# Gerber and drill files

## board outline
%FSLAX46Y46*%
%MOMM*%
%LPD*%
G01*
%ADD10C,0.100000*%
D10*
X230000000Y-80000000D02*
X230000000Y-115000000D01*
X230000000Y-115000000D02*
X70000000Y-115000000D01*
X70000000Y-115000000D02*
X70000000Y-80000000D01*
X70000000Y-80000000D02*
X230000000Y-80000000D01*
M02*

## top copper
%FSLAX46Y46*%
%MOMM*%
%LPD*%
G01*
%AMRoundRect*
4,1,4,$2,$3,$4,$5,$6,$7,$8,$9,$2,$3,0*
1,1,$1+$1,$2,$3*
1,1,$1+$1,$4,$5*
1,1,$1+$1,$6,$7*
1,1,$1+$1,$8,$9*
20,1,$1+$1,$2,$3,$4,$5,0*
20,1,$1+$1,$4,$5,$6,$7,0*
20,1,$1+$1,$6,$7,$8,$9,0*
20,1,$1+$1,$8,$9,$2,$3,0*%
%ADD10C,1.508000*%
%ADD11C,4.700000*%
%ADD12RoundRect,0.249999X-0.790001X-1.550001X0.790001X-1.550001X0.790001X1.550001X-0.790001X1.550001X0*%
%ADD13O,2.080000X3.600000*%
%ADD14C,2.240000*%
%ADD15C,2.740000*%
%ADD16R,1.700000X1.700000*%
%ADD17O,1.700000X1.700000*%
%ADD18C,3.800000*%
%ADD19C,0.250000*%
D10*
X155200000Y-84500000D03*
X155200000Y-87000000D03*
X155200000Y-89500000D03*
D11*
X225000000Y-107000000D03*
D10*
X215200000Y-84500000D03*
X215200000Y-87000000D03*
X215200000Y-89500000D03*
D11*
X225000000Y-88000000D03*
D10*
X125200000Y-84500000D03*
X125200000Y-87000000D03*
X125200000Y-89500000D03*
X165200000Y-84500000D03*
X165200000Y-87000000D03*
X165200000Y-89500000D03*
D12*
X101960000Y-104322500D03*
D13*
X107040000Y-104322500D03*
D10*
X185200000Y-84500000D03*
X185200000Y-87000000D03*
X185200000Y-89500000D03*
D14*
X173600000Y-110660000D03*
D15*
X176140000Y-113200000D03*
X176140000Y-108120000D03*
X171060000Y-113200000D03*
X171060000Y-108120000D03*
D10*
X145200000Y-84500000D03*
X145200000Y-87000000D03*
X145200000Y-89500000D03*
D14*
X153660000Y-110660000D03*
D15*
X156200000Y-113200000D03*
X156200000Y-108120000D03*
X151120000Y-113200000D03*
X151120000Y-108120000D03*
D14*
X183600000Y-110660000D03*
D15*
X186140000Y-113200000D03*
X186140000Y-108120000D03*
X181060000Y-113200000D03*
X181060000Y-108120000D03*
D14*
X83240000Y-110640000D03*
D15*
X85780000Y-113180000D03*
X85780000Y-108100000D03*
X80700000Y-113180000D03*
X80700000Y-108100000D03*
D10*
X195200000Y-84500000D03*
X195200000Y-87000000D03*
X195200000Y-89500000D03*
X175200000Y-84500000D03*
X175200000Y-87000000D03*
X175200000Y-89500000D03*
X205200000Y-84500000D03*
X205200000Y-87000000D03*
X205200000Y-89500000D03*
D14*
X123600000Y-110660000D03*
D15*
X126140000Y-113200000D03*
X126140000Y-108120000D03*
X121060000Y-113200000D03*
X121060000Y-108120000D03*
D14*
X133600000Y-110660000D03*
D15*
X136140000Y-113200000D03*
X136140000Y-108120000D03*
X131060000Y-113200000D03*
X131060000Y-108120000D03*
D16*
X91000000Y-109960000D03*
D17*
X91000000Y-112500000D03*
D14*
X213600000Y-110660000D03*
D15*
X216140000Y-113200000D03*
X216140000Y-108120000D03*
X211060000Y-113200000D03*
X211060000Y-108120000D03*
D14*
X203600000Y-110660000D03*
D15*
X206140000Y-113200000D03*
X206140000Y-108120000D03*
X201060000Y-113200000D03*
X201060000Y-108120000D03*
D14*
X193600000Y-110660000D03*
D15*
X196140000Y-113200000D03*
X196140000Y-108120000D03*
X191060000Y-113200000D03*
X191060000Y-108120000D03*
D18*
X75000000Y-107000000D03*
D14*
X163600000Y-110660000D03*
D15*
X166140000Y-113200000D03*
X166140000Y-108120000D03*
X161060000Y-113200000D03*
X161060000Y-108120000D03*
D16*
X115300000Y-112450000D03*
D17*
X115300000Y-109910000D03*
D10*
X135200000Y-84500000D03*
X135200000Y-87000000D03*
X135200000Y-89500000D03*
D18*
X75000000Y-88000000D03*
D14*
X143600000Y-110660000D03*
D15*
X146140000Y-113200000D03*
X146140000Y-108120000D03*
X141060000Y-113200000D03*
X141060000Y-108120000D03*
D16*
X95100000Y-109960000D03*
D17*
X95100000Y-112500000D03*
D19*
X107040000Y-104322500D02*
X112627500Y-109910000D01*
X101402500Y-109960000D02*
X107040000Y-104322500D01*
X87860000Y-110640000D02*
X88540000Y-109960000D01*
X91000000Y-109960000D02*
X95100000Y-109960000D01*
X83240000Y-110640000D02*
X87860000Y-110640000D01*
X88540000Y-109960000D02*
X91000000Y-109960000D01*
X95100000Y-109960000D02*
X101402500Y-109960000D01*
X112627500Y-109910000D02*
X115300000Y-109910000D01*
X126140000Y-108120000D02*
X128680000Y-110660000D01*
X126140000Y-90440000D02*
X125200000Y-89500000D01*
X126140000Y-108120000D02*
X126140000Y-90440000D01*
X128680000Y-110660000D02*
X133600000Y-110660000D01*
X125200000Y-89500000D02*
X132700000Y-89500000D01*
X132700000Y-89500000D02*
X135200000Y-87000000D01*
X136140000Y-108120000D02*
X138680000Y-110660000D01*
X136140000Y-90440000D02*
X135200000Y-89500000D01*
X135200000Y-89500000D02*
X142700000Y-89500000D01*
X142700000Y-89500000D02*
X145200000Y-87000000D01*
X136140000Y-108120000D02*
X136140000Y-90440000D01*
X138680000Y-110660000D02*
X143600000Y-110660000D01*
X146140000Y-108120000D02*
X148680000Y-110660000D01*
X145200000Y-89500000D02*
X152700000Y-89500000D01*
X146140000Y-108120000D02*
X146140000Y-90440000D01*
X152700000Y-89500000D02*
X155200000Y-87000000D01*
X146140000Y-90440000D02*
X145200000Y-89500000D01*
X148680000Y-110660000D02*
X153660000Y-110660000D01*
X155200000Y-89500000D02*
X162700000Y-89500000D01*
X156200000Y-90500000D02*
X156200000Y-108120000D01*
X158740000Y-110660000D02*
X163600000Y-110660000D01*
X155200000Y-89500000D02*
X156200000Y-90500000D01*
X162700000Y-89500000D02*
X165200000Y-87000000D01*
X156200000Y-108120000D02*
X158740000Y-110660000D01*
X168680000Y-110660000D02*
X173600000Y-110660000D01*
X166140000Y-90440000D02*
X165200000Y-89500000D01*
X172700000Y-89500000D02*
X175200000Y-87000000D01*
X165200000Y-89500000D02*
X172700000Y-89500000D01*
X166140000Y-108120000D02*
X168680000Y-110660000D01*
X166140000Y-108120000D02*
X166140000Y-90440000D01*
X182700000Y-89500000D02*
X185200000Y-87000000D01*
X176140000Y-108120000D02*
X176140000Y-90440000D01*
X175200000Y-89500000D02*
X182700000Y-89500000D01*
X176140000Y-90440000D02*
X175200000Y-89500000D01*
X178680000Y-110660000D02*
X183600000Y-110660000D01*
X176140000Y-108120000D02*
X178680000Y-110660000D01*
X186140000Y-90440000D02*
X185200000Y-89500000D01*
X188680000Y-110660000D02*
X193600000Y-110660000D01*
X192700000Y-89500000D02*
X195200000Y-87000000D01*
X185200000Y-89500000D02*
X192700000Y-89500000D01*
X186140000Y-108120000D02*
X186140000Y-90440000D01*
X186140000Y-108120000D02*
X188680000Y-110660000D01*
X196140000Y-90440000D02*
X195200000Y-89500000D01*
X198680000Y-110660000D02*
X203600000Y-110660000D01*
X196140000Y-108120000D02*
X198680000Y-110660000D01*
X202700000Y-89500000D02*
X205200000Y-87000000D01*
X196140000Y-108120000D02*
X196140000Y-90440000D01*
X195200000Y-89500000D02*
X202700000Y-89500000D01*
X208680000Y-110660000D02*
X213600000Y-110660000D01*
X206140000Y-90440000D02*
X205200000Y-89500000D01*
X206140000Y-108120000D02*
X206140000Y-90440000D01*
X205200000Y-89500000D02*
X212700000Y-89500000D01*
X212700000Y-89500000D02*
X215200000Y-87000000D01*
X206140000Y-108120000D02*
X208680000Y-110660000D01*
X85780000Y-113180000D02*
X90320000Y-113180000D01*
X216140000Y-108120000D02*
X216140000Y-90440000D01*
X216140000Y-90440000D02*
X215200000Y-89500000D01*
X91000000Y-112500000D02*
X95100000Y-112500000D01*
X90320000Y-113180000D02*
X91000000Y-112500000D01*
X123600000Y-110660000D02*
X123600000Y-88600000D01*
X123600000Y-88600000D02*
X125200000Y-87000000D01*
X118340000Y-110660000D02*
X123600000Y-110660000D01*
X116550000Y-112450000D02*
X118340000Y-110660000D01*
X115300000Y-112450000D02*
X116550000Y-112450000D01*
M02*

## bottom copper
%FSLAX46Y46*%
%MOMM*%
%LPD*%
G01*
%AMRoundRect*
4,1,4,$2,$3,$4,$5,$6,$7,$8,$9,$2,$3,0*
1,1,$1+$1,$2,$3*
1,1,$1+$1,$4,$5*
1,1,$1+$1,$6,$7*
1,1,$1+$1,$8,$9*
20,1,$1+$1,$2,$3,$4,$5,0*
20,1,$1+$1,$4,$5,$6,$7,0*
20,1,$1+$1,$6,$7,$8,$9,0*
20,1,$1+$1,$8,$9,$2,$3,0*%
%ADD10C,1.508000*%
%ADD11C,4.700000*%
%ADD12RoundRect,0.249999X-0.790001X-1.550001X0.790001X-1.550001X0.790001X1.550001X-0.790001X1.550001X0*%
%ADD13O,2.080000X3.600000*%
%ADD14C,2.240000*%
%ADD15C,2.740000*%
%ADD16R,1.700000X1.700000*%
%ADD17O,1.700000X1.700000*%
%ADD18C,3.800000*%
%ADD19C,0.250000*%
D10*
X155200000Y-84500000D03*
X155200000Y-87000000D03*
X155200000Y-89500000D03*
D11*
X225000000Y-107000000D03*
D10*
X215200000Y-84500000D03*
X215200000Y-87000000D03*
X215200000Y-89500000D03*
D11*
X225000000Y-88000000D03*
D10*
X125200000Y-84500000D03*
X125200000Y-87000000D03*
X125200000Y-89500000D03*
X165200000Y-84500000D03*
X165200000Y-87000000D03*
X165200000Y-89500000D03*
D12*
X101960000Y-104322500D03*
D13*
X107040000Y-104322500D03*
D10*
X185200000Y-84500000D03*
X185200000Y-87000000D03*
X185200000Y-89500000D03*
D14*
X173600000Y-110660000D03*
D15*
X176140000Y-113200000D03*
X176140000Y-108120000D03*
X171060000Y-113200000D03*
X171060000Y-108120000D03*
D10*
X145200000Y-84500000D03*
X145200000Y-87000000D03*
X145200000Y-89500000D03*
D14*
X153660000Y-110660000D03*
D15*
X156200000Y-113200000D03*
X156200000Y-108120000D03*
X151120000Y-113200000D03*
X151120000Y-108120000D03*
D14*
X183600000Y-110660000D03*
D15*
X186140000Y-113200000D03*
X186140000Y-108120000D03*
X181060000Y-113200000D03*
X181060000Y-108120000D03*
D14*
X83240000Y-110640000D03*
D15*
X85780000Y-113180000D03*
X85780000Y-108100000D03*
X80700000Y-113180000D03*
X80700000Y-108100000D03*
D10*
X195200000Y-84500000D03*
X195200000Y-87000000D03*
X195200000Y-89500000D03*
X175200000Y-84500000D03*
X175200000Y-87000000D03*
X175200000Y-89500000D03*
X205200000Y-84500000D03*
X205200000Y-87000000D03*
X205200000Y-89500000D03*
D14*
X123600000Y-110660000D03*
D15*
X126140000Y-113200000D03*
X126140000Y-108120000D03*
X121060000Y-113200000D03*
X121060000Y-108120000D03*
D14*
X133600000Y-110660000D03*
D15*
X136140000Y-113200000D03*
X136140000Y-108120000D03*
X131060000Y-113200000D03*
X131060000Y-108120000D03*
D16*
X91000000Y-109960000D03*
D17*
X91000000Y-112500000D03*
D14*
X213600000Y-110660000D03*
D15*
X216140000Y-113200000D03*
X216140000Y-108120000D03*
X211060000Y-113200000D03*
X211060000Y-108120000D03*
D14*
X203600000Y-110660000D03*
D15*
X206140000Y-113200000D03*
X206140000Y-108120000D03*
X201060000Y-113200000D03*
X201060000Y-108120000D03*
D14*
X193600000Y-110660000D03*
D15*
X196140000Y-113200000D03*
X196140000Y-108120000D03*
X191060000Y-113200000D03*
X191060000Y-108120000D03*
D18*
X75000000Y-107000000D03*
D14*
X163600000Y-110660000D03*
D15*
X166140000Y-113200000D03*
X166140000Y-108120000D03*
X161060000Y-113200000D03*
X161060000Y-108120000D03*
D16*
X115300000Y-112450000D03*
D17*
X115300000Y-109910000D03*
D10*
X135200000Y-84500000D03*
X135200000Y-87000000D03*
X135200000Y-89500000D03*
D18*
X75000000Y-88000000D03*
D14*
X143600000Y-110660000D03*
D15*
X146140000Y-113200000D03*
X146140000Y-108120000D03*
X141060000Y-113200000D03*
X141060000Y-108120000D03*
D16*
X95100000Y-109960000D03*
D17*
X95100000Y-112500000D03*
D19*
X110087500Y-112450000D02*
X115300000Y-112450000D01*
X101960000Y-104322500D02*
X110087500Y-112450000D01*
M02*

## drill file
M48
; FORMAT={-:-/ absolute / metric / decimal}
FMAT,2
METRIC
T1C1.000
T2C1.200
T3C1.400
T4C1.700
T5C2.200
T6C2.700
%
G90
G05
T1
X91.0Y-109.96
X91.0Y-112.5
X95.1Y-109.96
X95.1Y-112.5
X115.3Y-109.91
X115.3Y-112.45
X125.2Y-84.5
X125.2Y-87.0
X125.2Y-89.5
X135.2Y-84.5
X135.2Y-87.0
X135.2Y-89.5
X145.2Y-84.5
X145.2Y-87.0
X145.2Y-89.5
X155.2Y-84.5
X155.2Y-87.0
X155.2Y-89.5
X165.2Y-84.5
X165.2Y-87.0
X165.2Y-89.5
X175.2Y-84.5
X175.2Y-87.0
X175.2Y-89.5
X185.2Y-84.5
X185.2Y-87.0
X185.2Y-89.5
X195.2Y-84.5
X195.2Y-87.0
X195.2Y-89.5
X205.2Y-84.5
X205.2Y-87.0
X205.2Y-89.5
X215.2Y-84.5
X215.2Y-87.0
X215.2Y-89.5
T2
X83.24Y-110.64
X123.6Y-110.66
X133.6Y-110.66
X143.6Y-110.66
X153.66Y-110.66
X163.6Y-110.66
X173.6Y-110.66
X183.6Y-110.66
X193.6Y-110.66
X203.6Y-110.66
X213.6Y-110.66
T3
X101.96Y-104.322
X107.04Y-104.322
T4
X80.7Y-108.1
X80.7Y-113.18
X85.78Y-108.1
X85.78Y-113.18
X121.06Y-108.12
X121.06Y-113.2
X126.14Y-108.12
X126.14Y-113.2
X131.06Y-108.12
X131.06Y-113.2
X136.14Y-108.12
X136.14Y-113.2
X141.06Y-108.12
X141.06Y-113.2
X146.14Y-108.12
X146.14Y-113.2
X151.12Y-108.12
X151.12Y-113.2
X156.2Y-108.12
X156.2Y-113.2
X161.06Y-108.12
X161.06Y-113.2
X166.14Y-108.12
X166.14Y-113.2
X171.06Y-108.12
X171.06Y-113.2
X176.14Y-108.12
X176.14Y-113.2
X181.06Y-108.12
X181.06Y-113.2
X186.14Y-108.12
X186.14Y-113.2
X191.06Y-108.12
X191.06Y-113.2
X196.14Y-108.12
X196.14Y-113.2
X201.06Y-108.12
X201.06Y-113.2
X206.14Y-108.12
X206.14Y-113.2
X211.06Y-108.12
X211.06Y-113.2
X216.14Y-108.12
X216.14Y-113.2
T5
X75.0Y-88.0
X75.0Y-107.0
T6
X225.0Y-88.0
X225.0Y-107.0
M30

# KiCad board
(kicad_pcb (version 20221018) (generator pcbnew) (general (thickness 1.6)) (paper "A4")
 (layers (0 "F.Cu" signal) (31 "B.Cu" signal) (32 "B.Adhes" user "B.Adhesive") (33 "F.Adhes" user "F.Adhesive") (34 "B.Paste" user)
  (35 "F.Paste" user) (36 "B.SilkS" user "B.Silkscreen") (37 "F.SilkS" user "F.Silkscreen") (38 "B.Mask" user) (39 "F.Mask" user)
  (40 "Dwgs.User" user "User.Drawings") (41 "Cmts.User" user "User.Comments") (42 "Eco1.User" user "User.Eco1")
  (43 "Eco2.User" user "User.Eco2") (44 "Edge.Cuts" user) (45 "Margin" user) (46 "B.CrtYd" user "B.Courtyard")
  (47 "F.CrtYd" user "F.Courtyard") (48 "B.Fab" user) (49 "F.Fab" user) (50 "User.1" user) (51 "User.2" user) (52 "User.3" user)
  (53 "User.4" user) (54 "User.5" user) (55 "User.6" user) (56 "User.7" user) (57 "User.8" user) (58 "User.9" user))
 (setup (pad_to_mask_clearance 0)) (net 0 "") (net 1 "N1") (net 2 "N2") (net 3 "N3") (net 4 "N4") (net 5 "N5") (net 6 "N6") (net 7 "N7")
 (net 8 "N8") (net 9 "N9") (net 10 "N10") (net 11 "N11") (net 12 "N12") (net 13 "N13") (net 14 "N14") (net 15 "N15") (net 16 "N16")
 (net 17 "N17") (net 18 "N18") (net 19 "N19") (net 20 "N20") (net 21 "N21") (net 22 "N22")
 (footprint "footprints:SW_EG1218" (layer "F.Cu") (at 155.2 87 -90)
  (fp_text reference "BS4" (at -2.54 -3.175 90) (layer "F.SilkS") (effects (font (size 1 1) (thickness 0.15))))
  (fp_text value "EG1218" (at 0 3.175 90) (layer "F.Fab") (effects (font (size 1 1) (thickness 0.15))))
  (pad "1" thru_hole circle (at -2.5 0 270) (size 1.508 1.508) (drill 1) (layers "*.Cu" "*.Mask") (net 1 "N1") (solder_mask_margin 0.102))
  (pad "2" thru_hole circle (at 0 0 270) (size 1.508 1.508) (drill 1) (layers "*.Cu" "*.Mask") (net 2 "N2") (solder_mask_margin 0.102))
  (pad "3" thru_hole circle (at 2.5 0 270) (size 1.508 1.508) (drill 1) (layers "*.Cu" "*.Mask") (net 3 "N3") (solder_mask_margin 0.102)))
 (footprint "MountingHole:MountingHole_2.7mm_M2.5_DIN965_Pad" (layer "F.Cu") (at 225 107)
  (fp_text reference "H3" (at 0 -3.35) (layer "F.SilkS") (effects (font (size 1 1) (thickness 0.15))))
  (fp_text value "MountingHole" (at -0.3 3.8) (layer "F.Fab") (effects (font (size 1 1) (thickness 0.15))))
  (pad "1" thru_hole circle (at 0 0) (size 4.7 4.7) (drill 2.7) (layers "*.Cu" "*.Mask")))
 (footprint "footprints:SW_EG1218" (layer "F.Cu") (at 215.2 87 -90)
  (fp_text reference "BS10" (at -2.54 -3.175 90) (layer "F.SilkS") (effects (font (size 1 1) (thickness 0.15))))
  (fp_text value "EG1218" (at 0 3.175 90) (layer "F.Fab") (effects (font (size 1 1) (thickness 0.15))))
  (pad "1" thru_hole circle (at -2.5 0 270) (size 1.508 1.508) (drill 1) (layers "*.Cu" "*.Mask") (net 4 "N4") (solder_mask_margin 0.102))
  (pad "2" thru_hole circle (at 0 0 270) (size 1.508 1.508) (drill 1) (layers "*.Cu" "*.Mask") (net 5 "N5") (solder_mask_margin 0.102))
  (pad "3" thru_hole circle (at 2.5 0 270) (size 1.508 1.508) (drill 1) (layers "*.Cu" "*.Mask") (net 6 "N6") (solder_mask_margin 0.102)))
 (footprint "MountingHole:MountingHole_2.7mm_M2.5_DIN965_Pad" (layer "F.Cu") (at 225 88)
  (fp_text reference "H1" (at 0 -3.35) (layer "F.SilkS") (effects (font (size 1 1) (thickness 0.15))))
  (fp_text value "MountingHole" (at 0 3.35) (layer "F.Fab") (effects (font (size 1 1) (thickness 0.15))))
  (pad "1" thru_hole circle (at 0 0) (size 4.7 4.7) (drill 2.7) (layers "*.Cu" "*.Mask")))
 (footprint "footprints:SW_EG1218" (layer "F.Cu") (at 125.2 87 -90)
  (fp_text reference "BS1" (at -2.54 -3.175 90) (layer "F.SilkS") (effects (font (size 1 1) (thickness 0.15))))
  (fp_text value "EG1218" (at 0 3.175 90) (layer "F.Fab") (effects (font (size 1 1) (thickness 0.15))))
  (pad "1" thru_hole circle (at -2.5 0 270) (size 1.508 1.508) (drill 1) (layers "*.Cu" "*.Mask") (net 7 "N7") (solder_mask_margin 0.102))
  (pad "2" thru_hole circle (at 0 0 270) (size 1.508 1.508) (drill 1) (layers "*.Cu" "*.Mask") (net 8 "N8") (solder_mask_margin 0.102))
  (pad "3" thru_hole circle (at 2.5 0 270) (size 1.508 1.508) (drill 1) (layers "*.Cu" "*.Mask") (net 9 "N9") (solder_mask_margin 0.102)))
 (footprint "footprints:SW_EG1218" (layer "F.Cu") (at 165.2 87 -90)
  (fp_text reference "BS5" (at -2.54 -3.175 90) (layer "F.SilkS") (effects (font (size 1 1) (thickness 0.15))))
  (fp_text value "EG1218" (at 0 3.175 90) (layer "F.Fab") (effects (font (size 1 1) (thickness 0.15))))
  (pad "1" thru_hole circle (at -2.5 0 270) (size 1.508 1.508) (drill 1) (layers "*.Cu" "*.Mask") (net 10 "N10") (solder_mask_margin 0.102))
  (pad "2" thru_hole circle (at 0 0 270) (size 1.508 1.508) (drill 1) (layers "*.Cu" "*.Mask") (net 3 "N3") (solder_mask_margin 0.102))
  (pad "3" thru_hole circle (at 2.5 0 270) (size 1.508 1.508) (drill 1) (layers "*.Cu" "*.Mask") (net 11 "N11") (solder_mask_margin 0.102)))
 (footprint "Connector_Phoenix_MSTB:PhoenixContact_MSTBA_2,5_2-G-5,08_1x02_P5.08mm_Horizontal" (layer "F.Cu") (at 101.96 104.3225)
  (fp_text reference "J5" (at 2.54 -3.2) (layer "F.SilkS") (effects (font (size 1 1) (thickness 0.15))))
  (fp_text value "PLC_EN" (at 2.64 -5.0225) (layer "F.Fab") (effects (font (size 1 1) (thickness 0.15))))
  (pad "1" thru_hole roundrect (at 0 0) (size 2.08 3.6) (drill 1.4) (layers "*.Cu" "*.Mask") (roundrect_rratio 0.1201918269) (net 8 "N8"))
  (pad "2" thru_hole oval (at 5.08 0) (size 2.08 3.6) (drill 1.4) (layers "*.Cu" "*.Mask") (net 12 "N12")))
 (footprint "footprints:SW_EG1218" (layer "F.Cu") (at 185.2 87 -90)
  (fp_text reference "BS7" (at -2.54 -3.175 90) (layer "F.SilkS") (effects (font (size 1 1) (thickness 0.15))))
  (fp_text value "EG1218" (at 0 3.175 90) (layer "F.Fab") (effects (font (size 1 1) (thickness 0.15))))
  (pad "1" thru_hole circle (at -2.5 0 270) (size 1.508 1.508) (drill 1) (layers "*.Cu" "*.Mask") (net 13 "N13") (solder_mask_margin 0.102))
  (pad "2" thru_hole circle (at 0 0 270) (size 1.508 1.508) (drill 1) (layers "*.Cu" "*.Mask") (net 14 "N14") (solder_mask_margin 0.102))
  (pad "3" thru_hole circle (at 2.5 0 270) (size 1.508 1.508) (drill 1) (layers "*.Cu" "*.Mask") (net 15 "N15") (solder_mask_margin 0.102)))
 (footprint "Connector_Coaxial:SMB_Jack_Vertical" (layer "F.Cu") (at 173.6 110.66 180)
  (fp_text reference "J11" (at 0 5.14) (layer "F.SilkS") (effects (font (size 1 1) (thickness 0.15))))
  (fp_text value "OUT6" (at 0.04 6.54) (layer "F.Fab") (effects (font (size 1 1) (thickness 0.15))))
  (pad "1" thru_hole circle (at 0 0 180) (size 2.24 2.24) (drill 1.2) (layers "*.Cu" "*.Mask") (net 11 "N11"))
  (pad "2" thru_hole circle (at -2.54 -2.54 180) (size 2.74 2.74) (drill 1.7) (layers "*.Cu" "*.Mask") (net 14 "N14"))
  (pad "2" thru_hole circle (at -2.54 2.54 180) (size 2.74 2.74) (drill 1.7) (layers "*.Cu" "*.Mask") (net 14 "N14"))
  (pad "2" thru_hole circle (at 2.54 -2.54 180) (size 2.74 2.74) (drill 1.7) (layers "*.Cu" "*.Mask") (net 14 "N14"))
  (pad "2" thru_hole circle (at 2.54 2.54 180) (size 2.74 2.74) (drill 1.7) (layers "*.Cu" "*.Mask") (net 14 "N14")))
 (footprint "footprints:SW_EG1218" (layer "F.Cu") (at 145.2 87 -90)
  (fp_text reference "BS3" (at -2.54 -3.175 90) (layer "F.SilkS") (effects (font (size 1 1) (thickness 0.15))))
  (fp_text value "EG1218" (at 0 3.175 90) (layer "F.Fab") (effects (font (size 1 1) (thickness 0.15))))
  (pad "1" thru_hole circle (at -2.5 0 270) (size 1.508 1.508) (drill 1) (layers "*.Cu" "*.Mask") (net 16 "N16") (solder_mask_margin 0.102))
  (pad "2" thru_hole circle (at 0 0 270) (size 1.508 1.508) (drill 1) (layers "*.Cu" "*.Mask") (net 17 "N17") (solder_mask_margin 0.102))
  (pad "3" thru_hole circle (at 2.5 0 270) (size 1.508 1.508) (drill 1) (layers "*.Cu" "*.Mask") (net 2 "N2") (solder_mask_margin 0.102)))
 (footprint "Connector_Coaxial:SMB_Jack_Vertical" (layer "F.Cu") (at 153.66 110.66 180)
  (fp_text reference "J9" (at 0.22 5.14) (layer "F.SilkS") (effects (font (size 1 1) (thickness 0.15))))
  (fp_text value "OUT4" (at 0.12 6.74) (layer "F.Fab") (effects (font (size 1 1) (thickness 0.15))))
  (pad "1" thru_hole circle (at 0 0 180) (size 2.24 2.24) (drill 1.2) (layers "*.Cu" "*.Mask") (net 2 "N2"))
  (pad "2" thru_hole circle (at -2.54 -2.54 180) (size 2.74 2.74) (drill 1.7) (layers "*.Cu" "*.Mask") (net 3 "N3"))
  (pad "2" thru_hole circle (at -2.54 2.54 180) (size 2.74 2.74) (drill 1.7) (layers "*.Cu" "*.Mask") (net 3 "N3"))
  (pad "2" thru_hole circle (at 2.54 -2.54 180) (size 2.74 2.74) (drill 1.7) (layers "*.Cu" "*.Mask") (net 3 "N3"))
  (pad "2" thru_hole circle (at 2.54 2.54 180) (size 2.74 2.74) (drill 1.7) (layers "*.Cu" "*.Mask") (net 3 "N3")))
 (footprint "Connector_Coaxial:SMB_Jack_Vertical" (layer "F.Cu") (at 183.6 110.66 180)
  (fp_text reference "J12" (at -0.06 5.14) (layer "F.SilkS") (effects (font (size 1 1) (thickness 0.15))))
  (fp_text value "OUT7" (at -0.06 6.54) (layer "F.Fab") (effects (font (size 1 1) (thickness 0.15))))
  (pad "1" thru_hole circle (at 0 0 180) (size 2.24 2.24) (drill 1.2) (layers "*.Cu" "*.Mask") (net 14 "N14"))
  (pad "2" thru_hole circle (at -2.54 -2.54 180) (size 2.74 2.74) (drill 1.7) (layers "*.Cu" "*.Mask") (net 15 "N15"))
  (pad "2" thru_hole circle (at -2.54 2.54 180) (size 2.74 2.74) (drill 1.7) (layers "*.Cu" "*.Mask") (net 15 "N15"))
  (pad "2" thru_hole circle (at 2.54 -2.54 180) (size 2.74 2.74) (drill 1.7) (layers "*.Cu" "*.Mask") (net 15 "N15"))
  (pad "2" thru_hole circle (at 2.54 2.54 180) (size 2.74 2.74) (drill 1.7) (layers "*.Cu" "*.Mask") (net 15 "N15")))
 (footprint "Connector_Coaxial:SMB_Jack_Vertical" (layer "F.Cu") (at 83.24 110.64 180)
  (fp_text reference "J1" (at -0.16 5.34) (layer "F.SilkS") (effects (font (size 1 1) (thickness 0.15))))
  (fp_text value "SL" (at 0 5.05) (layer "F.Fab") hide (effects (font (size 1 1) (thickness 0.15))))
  (pad "1" thru_hole circle (at 0 0 180) (size 2.24 2.24) (drill 1.2) (layers "*.Cu" "*.Mask") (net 12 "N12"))
  (pad "2" thru_hole circle (at -2.54 -2.54 180) (size 2.74 2.74) (drill 1.7) (layers "*.Cu" "*.Mask") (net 6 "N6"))
  (pad "2" thru_hole circle (at -2.54 2.54 180) (size 2.74 2.74) (drill 1.7) (layers "*.Cu" "*.Mask") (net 6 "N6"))
  (pad "2" thru_hole circle (at 2.54 -2.54 180) (size 2.74 2.74) (drill 1.7) (layers "*.Cu" "*.Mask") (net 6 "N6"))
  (pad "2" thru_hole circle (at 2.54 2.54 180) (size 2.74 2.74) (drill 1.7) (layers "*.Cu" "*.Mask") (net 6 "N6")))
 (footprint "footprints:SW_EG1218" (layer "F.Cu") (at 195.2 87 -90)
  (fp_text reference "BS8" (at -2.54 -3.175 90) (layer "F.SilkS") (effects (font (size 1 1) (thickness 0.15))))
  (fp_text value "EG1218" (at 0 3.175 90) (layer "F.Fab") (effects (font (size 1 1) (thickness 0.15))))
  (pad "1" thru_hole circle (at -2.5 0 270) (size 1.508 1.508) (drill 1) (layers "*.Cu" "*.Mask") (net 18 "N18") (solder_mask_margin 0.102))
  (pad "2" thru_hole circle (at 0 0 270) (size 1.508 1.508) (drill 1) (layers "*.Cu" "*.Mask") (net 15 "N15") (solder_mask_margin 0.102))
  (pad "3" thru_hole circle (at 2.5 0 270) (size 1.508 1.508) (drill 1) (layers "*.Cu" "*.Mask") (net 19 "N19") (solder_mask_margin 0.102)))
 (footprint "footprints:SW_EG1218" (layer "F.Cu") (at 175.2 87 -90)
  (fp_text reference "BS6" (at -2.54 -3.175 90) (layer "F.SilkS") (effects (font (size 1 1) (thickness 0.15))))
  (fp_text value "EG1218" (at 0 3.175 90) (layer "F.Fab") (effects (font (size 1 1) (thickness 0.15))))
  (pad "1" thru_hole circle (at -2.5 0 270) (size 1.508 1.508) (drill 1) (layers "*.Cu" "*.Mask") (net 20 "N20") (solder_mask_margin 0.102))
  (pad "2" thru_hole circle (at 0 0 270) (size 1.508 1.508) (drill 1) (layers "*.Cu" "*.Mask") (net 11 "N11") (solder_mask_margin 0.102))
  (pad "3" thru_hole circle (at 2.5 0 270) (size 1.508 1.508) (drill 1) (layers "*.Cu" "*.Mask") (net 14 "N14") (solder_mask_margin 0.102)))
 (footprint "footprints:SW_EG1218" (layer "F.Cu") (at 205.2 87 -90)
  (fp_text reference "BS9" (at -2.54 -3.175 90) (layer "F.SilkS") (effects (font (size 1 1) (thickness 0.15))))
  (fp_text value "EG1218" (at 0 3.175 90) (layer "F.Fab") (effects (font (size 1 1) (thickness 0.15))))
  (pad "1" thru_hole circle (at -2.5 0 270) (size 1.508 1.508) (drill 1) (layers "*.Cu" "*.Mask") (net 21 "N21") (solder_mask_margin 0.102))
  (pad "2" thru_hole circle (at 0 0 270) (size 1.508 1.508) (drill 1) (layers "*.Cu" "*.Mask") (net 19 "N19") (solder_mask_margin 0.102))
  (pad "3" thru_hole circle (at 2.5 0 270) (size 1.508 1.508) (drill 1) (layers "*.Cu" "*.Mask") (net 5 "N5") (solder_mask_margin 0.102)))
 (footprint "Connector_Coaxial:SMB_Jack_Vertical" (layer "F.Cu") (at 123.6 110.66 180)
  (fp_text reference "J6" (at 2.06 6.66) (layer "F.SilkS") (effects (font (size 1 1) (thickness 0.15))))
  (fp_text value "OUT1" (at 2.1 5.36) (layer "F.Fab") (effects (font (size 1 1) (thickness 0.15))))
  (pad "1" thru_hole circle (at 0 0 180) (size 2.24 2.24) (drill 1.2) (layers "*.Cu" "*.Mask") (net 8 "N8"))
  (pad "2" thru_hole circle (at -2.54 -2.54 180) (size 2.74 2.74) (drill 1.7) (layers "*.Cu" "*.Mask") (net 9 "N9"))
  (pad "2" thru_hole circle (at -2.54 2.54 180) (size 2.74 2.74) (drill 1.7) (layers "*.Cu" "*.Mask") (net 9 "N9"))
  (pad "2" thru_hole circle (at 2.54 -2.54 180) (size 2.74 2.74) (drill 1.7) (layers "*.Cu" "*.Mask") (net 9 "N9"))
  (pad "2" thru_hole circle (at 2.54 2.54 180) (size 2.74 2.74) (drill 1.7) (layers "*.Cu" "*.Mask") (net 9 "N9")))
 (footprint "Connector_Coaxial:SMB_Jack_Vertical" (layer "F.Cu") (at 133.6 110.66 180)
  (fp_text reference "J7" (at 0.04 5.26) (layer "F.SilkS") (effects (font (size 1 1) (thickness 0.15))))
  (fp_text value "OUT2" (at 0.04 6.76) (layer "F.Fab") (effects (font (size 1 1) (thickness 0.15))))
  (pad "1" thru_hole circle (at 0 0 180) (size 2.24 2.24) (drill 1.2) (layers "*.Cu" "*.Mask") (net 9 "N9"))
  (pad "2" thru_hole circle (at -2.54 -2.54 180) (size 2.74 2.74) (drill 1.7) (layers "*.Cu" "*.Mask") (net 17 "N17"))
  (pad "2" thru_hole circle (at -2.54 2.54 180) (size 2.74 2.74) (drill 1.7) (layers "*.Cu" "*.Mask") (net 17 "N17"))
  (pad "2" thru_hole circle (at 2.54 -2.54 180) (size 2.74 2.74) (drill 1.7) (layers "*.Cu" "*.Mask") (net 17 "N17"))
  (pad "2" thru_hole circle (at 2.54 2.54 180) (size 2.74 2.74) (drill 1.7) (layers "*.Cu" "*.Mask") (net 17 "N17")))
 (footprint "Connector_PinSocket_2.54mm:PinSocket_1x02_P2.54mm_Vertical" (layer "F.Cu") (at 91 109.96)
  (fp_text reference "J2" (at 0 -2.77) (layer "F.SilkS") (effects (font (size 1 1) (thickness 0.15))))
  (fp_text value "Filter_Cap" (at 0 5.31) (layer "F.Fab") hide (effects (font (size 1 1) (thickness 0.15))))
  (pad "1" thru_hole rect (at 0 0) (size 1.7 1.7) (drill 1) (layers "*.Cu" "*.Mask") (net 12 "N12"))
  (pad "2" thru_hole oval (at 0 2.54) (size 1.7 1.7) (drill 1) (layers "*.Cu" "*.Mask") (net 6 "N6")))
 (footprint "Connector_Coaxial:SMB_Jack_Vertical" (layer "F.Cu") (at 213.6 110.66 180)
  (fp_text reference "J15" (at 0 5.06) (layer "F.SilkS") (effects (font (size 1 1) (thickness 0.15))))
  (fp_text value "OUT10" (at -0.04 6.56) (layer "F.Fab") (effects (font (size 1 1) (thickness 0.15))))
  (pad "1" thru_hole circle (at 0 0 180) (size 2.24 2.24) (drill 1.2) (layers "*.Cu" "*.Mask") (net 5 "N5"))
  (pad "2" thru_hole circle (at -2.54 -2.54 180) (size 2.74 2.74) (drill 1.7) (layers "*.Cu" "*.Mask") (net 6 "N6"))
  (pad "2" thru_hole circle (at -2.54 2.54 180) (size 2.74 2.74) (drill 1.7) (layers "*.Cu" "*.Mask") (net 6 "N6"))
  (pad "2" thru_hole circle (at 2.54 -2.54 180) (size 2.74 2.74) (drill 1.7) (layers "*.Cu" "*.Mask") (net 6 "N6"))
  (pad "2" thru_hole circle (at 2.54 2.54 180) (size 2.74 2.74) (drill 1.7) (layers "*.Cu" "*.Mask") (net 6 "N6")))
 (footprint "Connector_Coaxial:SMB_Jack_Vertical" (layer "F.Cu") (at 203.6 110.66 180)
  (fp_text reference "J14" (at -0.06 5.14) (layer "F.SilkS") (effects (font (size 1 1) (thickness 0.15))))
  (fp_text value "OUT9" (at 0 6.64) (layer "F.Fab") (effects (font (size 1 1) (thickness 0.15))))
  (pad "1" thru_hole circle (at 0 0 180) (size 2.24 2.24) (drill 1.2) (layers "*.Cu" "*.Mask") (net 19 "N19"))
  (pad "2" thru_hole circle (at -2.54 -2.54 180) (size 2.74 2.74) (drill 1.7) (layers "*.Cu" "*.Mask") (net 5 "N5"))
  (pad "2" thru_hole circle (at -2.54 2.54 180) (size 2.74 2.74) (drill 1.7) (layers "*.Cu" "*.Mask") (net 5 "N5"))
  (pad "2" thru_hole circle (at 2.54 -2.54 180) (size 2.74 2.74) (drill 1.7) (layers "*.Cu" "*.Mask") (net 5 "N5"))
  (pad "2" thru_hole circle (at 2.54 2.54 180) (size 2.74 2.74) (drill 1.7) (layers "*.Cu" "*.Mask") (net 5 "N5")))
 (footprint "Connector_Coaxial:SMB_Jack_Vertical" (layer "F.Cu") (at 193.6 110.66 180)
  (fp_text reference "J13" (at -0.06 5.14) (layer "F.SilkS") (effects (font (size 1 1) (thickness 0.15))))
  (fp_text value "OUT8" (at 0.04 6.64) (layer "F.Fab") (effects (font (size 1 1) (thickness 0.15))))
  (pad "1" thru_hole circle (at 0 0 180) (size 2.24 2.24) (drill 1.2) (layers "*.Cu" "*.Mask") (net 15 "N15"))
  (pad "2" thru_hole circle (at -2.54 -2.54 180) (size 2.74 2.74) (drill 1.7) (layers "*.Cu" "*.Mask") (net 19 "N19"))
  (pad "2" thru_hole circle (at -2.54 2.54 180) (size 2.74 2.74) (drill 1.7) (layers "*.Cu" "*.Mask") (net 19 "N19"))
  (pad "2" thru_hole circle (at 2.54 -2.54 180) (size 2.74 2.74) (drill 1.7) (layers "*.Cu" "*.Mask") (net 19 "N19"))
  (pad "2" thru_hole circle (at 2.54 2.54 180) (size 2.74 2.74) (drill 1.7) (layers "*.Cu" "*.Mask") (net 19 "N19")))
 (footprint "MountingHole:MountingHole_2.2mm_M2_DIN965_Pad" (layer "F.Cu") (at 75 107)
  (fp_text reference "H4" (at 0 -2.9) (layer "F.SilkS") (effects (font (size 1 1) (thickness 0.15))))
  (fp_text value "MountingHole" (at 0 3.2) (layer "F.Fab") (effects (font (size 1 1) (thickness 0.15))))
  (pad "1" thru_hole circle (at 0 0) (size 3.8 3.8) (drill 2.2) (layers "*.Cu" "*.Mask")))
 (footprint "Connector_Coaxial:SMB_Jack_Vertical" (layer "F.Cu") (at 163.6 110.66 180)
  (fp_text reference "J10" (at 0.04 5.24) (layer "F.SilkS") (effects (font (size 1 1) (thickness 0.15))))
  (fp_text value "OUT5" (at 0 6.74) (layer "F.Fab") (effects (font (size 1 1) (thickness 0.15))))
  (pad "1" thru_hole circle (at 0 0 180) (size 2.24 2.24) (drill 1.2) (layers "*.Cu" "*.Mask") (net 3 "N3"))
  (pad "2" thru_hole circle (at -2.54 -2.54 180) (size 2.74 2.74) (drill 1.7) (layers "*.Cu" "*.Mask") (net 11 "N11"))
  (pad "2" thru_hole circle (at -2.54 2.54 180) (size 2.74 2.74) (drill 1.7) (layers "*.Cu" "*.Mask") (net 11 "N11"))
  (pad "2" thru_hole circle (at 2.54 -2.54 180) (size 2.74 2.74) (drill 1.7) (layers "*.Cu" "*.Mask") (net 11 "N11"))
  (pad "2" thru_hole circle (at 2.54 2.54 180) (size 2.74 2.74) (drill 1.7) (layers "*.Cu" "*.Mask") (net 11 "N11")))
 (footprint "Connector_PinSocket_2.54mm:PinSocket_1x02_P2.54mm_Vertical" (layer "F.Cu") (at 115.3 112.45 180)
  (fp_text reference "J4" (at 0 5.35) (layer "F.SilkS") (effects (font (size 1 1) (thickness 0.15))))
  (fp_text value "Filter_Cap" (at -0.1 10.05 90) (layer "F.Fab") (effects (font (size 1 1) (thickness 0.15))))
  (pad "1" thru_hole rect (at 0 0 180) (size 1.7 1.7) (drill 1) (layers "*.Cu" "*.Mask") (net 8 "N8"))
  (pad "2" thru_hole oval (at 0 2.54 180) (size 1.7 1.7) (drill 1) (layers "*.Cu" "*.Mask") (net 12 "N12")))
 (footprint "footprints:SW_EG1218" (layer "F.Cu") (at 135.2 87 -90)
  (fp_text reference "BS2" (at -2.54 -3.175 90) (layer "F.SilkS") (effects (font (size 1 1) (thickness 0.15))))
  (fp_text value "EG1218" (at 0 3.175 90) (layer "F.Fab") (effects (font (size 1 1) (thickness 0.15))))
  (pad "1" thru_hole circle (at -2.5 0 270) (size 1.508 1.508) (drill 1) (layers "*.Cu" "*.Mask") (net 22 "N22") (solder_mask_margin 0.102))
  (pad "2" thru_hole circle (at 0 0 270) (size 1.508 1.508) (drill 1) (layers "*.Cu" "*.Mask") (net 9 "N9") (solder_mask_margin 0.102))
  (pad "3" thru_hole circle (at 2.5 0 270) (size 1.508 1.508) (drill 1) (layers "*.Cu" "*.Mask") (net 17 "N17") (solder_mask_margin 0.102)))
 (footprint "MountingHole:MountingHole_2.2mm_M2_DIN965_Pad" (layer "F.Cu") (at 75 88)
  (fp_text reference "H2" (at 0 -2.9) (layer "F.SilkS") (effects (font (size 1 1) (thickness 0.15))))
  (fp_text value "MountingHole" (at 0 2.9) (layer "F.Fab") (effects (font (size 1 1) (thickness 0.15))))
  (pad "1" thru_hole circle (at 0 0) (size 3.8 3.8) (drill 2.2) (layers "*.Cu" "*.Mask")))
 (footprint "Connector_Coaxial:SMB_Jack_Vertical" (layer "F.Cu") (at 143.6 110.66 180)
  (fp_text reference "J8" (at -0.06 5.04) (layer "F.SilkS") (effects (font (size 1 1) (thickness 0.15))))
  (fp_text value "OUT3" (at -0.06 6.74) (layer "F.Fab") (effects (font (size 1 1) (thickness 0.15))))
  (pad "1" thru_hole circle (at 0 0 180) (size 2.24 2.24) (drill 1.2) (layers "*.Cu" "*.Mask") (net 17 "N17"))
  (pad "2" thru_hole circle (at -2.54 -2.54 180) (size 2.74 2.74) (drill 1.7) (layers "*.Cu" "*.Mask") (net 2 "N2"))
  (pad "2" thru_hole circle (at -2.54 2.54 180) (size 2.74 2.74) (drill 1.7) (layers "*.Cu" "*.Mask") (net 2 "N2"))
  (pad "2" thru_hole circle (at 2.54 -2.54 180) (size 2.74 2.74) (drill 1.7) (layers "*.Cu" "*.Mask") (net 2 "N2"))
  (pad "2" thru_hole circle (at 2.54 2.54 180) (size 2.74 2.74) (drill 1.7) (layers "*.Cu" "*.Mask") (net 2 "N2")))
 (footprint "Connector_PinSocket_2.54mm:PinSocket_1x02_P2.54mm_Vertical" (layer "F.Cu") (at 95.1 109.96)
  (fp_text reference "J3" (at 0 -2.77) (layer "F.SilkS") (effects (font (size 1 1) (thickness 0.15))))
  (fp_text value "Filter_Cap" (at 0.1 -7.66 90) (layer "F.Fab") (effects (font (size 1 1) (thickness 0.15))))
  (pad "1" thru_hole rect (at 0 0) (size 1.7 1.7) (drill 1) (layers "*.Cu" "*.Mask") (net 12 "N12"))
  (pad "2" thru_hole oval (at 0 2.54) (size 1.7 1.7) (drill 1) (layers "*.Cu" "*.Mask") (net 6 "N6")))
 (gr_line (start 230 80) (end 230 115) (stroke (width 0.1) (type default)) (layer "Edge.Cuts"))
 (gr_line (start 230 115) (end 70 115) (stroke (width 0.1) (type default)) (layer "Edge.Cuts"))
 (gr_line (start 70 115) (end 70 80) (stroke (width 0.1) (type default)) (layer "Edge.Cuts"))
 (gr_line (start 70 80) (end 230 80) (stroke (width 0.1) (type default)) (layer "Edge.Cuts"))
 (segment (start 107.04 104.3225) (end 112.6275 109.91) (width 0.25) (layer "F.Cu") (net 12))
 (segment (start 101.4025 109.96) (end 107.04 104.3225) (width 0.25) (layer "F.Cu") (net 12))
 (segment (start 87.86 110.64) (end 88.54 109.96) (width 0.25) (layer "F.Cu") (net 12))
 (segment (start 91 109.96) (end 95.1 109.96) (width 0.25) (layer "F.Cu") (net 12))
 (segment (start 83.24 110.64) (end 87.86 110.64) (width 0.25) (layer "F.Cu") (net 12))
 (segment (start 88.54 109.96) (end 91 109.96) (width 0.25) (layer "F.Cu") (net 12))
 (segment (start 95.1 109.96) (end 101.4025 109.96) (width 0.25) (layer "F.Cu") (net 12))
 (segment (start 112.6275 109.91) (end 115.3 109.91) (width 0.25) (layer "F.Cu") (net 12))
 (segment (start 126.14 108.12) (end 128.68 110.66) (width 0.25) (layer "F.Cu") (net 9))
 (segment (start 126.14 90.44) (end 125.2 89.5) (width 0.25) (layer "F.Cu") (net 9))
 (segment (start 126.14 108.12) (end 126.14 90.44) (width 0.25) (layer "F.Cu") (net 9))
 (segment (start 128.68 110.66) (end 133.6 110.66) (width 0.25) (layer "F.Cu") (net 9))
 (segment (start 125.2 89.5) (end 132.7 89.5) (width 0.25) (layer "F.Cu") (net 9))
 (segment (start 132.7 89.5) (end 135.2 87) (width 0.25) (layer "F.Cu") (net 9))
 (segment (start 136.14 108.12) (end 138.68 110.66) (width 0.25) (layer "F.Cu") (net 17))
 (segment (start 136.14 90.44) (end 135.2 89.5) (width 0.25) (layer "F.Cu") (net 17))
 (segment (start 135.2 89.5) (end 142.7 89.5) (width 0.25) (layer "F.Cu") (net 17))
 (segment (start 142.7 89.5) (end 145.2 87) (width 0.25) (layer "F.Cu") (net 17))
 (segment (start 136.14 108.12) (end 136.14 90.44) (width 0.25) (layer "F.Cu") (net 17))
 (segment (start 138.68 110.66) (end 143.6 110.66) (width 0.25) (layer "F.Cu") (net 17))
 (segment (start 146.14 108.12) (end 148.68 110.66) (width 0.25) (layer "F.Cu") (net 2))
 (segment (start 145.2 89.5) (end 152.7 89.5) (width 0.25) (layer "F.Cu") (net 2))
 (segment (start 146.14 108.12) (end 146.14 90.44) (width 0.25) (layer "F.Cu") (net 2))
 (segment (start 152.7 89.5) (end 155.2 87) (width 0.25) (layer "F.Cu") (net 2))
 (segment (start 146.14 90.44) (end 145.2 89.5) (width 0.25) (layer "F.Cu") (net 2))
 (segment (start 148.68 110.66) (end 153.66 110.66) (width 0.25) (layer "F.Cu") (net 2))
 (segment (start 155.2 89.5) (end 162.7 89.5) (width 0.25) (layer "F.Cu") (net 3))
 (segment (start 156.2 90.5) (end 156.2 108.12) (width 0.25) (layer "F.Cu") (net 3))
 (segment (start 158.74 110.66) (end 163.6 110.66) (width 0.25) (layer "F.Cu") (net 3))
 (segment (start 155.2 89.5) (end 156.2 90.5) (width 0.25) (layer "F.Cu") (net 3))
 (segment (start 162.7 89.5) (end 165.2 87) (width 0.25) (layer "F.Cu") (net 3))
 (segment (start 156.2 108.12) (end 158.74 110.66) (width 0.25) (layer "F.Cu") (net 3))
 (segment (start 168.68 110.66) (end 173.6 110.66) (width 0.25) (layer "F.Cu") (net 11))
 (segment (start 166.14 90.44) (end 165.2 89.5) (width 0.25) (layer "F.Cu") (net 11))
 (segment (start 172.7 89.5) (end 175.2 87) (width 0.25) (layer "F.Cu") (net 11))
 (segment (start 165.2 89.5) (end 172.7 89.5) (width 0.25) (layer "F.Cu") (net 11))
 (segment (start 166.14 108.12) (end 168.68 110.66) (width 0.25) (layer "F.Cu") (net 11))
 (segment (start 166.14 108.12) (end 166.14 90.44) (width 0.25) (layer "F.Cu") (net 11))
 (segment (start 182.7 89.5) (end 185.2 87) (width 0.25) (layer "F.Cu") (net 14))
 (segment (start 176.14 108.12) (end 176.14 90.44) (width 0.25) (layer "F.Cu") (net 14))
 (segment (start 175.2 89.5) (end 182.7 89.5) (width 0.25) (layer "F.Cu") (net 14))
 (segment (start 176.14 90.44) (end 175.2 89.5) (width 0.25) (layer "F.Cu") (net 14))
 (segment (start 178.68 110.66) (end 183.6 110.66) (width 0.25) (layer "F.Cu") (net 14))
 (segment (start 176.14 108.12) (end 178.68 110.66) (width 0.25) (layer "F.Cu") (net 14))
 (segment (start 186.14 90.44) (end 185.2 89.5) (width 0.25) (layer "F.Cu") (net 15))
 (segment (start 188.68 110.66) (end 193.6 110.66) (width 0.25) (layer "F.Cu") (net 15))
 (segment (start 192.7 89.5) (end 195.2 87) (width 0.25) (layer "F.Cu") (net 15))
 (segment (start 185.2 89.5) (end 192.7 89.5) (width 0.25) (layer "F.Cu") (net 15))
 (segment (start 186.14 108.12) (end 186.14 90.44) (width 0.25) (layer "F.Cu") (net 15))
 (segment (start 186.14 108.12) (end 188.68 110.66) (width 0.25) (layer "F.Cu") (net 15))
 (segment (start 196.14 90.44) (end 195.2 89.5) (width 0.25) (layer "F.Cu") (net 19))
 (segment (start 198.68 110.66) (end 203.6 110.66) (width 0.25) (layer "F.Cu") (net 19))
 (segment (start 196.14 108.12) (end 198.68 110.66) (width 0.25) (layer "F.Cu") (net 19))
 (segment (start 202.7 89.5) (end 205.2 87) (width 0.25) (layer "F.Cu") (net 19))
 (segment (start 196.14 108.12) (end 196.14 90.44) (width 0.25) (layer "F.Cu") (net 19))
 (segment (start 195.2 89.5) (end 202.7 89.5) (width 0.25) (layer "F.Cu") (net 19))
 (segment (start 208.68 110.66) (end 213.6 110.66) (width 0.25) (layer "F.Cu") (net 5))
 (segment (start 206.14 90.44) (end 205.2 89.5) (width 0.25) (layer "F.Cu") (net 5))
 (segment (start 206.14 108.12) (end 206.14 90.44) (width 0.25) (layer "F.Cu") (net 5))
 (segment (start 205.2 89.5) (end 212.7 89.5) (width 0.25) (layer "F.Cu") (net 5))
 (segment (start 212.7 89.5) (end 215.2 87) (width 0.25) (layer "F.Cu") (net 5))
 (segment (start 206.14 108.12) (end 208.68 110.66) (width 0.25) (layer "F.Cu") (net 5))
 (segment (start 85.78 113.18) (end 90.32 113.18) (width 0.25) (layer "F.Cu") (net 6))
 (segment (start 216.14 108.12) (end 216.14 90.44) (width 0.25) (layer "F.Cu") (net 6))
 (segment (start 216.14 90.44) (end 215.2 89.5) (width 0.25) (layer "F.Cu") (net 6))
 (segment (start 91 112.5) (end 95.1 112.5) (width 0.25) (layer "F.Cu") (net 6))
 (segment (start 90.32 113.18) (end 91 112.5) (width 0.25) (layer "F.Cu") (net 6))
 (segment (start 123.6 110.66) (end 123.6 88.6) (width 0.25) (layer "F.Cu") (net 8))
 (segment (start 123.6 88.6) (end 125.2 87) (width 0.25) (layer "F.Cu") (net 8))
 (segment (start 118.34 110.66) (end 123.6 110.66) (width 0.25) (layer "F.Cu") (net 8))
 (segment (start 116.55 112.45) (end 118.34 110.66) (width 0.25) (layer "F.Cu") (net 8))
 (segment (start 115.3 112.45) (end 116.55 112.45) (width 0.25) (layer "F.Cu") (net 8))
 (segment (start 110.0875 112.45) (end 115.3 112.45) (width 0.25) (layer "B.Cu") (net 8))
 (segment (start 101.96 104.3225) (end 110.0875 112.45) (width 0.25) (layer "B.Cu") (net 8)))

